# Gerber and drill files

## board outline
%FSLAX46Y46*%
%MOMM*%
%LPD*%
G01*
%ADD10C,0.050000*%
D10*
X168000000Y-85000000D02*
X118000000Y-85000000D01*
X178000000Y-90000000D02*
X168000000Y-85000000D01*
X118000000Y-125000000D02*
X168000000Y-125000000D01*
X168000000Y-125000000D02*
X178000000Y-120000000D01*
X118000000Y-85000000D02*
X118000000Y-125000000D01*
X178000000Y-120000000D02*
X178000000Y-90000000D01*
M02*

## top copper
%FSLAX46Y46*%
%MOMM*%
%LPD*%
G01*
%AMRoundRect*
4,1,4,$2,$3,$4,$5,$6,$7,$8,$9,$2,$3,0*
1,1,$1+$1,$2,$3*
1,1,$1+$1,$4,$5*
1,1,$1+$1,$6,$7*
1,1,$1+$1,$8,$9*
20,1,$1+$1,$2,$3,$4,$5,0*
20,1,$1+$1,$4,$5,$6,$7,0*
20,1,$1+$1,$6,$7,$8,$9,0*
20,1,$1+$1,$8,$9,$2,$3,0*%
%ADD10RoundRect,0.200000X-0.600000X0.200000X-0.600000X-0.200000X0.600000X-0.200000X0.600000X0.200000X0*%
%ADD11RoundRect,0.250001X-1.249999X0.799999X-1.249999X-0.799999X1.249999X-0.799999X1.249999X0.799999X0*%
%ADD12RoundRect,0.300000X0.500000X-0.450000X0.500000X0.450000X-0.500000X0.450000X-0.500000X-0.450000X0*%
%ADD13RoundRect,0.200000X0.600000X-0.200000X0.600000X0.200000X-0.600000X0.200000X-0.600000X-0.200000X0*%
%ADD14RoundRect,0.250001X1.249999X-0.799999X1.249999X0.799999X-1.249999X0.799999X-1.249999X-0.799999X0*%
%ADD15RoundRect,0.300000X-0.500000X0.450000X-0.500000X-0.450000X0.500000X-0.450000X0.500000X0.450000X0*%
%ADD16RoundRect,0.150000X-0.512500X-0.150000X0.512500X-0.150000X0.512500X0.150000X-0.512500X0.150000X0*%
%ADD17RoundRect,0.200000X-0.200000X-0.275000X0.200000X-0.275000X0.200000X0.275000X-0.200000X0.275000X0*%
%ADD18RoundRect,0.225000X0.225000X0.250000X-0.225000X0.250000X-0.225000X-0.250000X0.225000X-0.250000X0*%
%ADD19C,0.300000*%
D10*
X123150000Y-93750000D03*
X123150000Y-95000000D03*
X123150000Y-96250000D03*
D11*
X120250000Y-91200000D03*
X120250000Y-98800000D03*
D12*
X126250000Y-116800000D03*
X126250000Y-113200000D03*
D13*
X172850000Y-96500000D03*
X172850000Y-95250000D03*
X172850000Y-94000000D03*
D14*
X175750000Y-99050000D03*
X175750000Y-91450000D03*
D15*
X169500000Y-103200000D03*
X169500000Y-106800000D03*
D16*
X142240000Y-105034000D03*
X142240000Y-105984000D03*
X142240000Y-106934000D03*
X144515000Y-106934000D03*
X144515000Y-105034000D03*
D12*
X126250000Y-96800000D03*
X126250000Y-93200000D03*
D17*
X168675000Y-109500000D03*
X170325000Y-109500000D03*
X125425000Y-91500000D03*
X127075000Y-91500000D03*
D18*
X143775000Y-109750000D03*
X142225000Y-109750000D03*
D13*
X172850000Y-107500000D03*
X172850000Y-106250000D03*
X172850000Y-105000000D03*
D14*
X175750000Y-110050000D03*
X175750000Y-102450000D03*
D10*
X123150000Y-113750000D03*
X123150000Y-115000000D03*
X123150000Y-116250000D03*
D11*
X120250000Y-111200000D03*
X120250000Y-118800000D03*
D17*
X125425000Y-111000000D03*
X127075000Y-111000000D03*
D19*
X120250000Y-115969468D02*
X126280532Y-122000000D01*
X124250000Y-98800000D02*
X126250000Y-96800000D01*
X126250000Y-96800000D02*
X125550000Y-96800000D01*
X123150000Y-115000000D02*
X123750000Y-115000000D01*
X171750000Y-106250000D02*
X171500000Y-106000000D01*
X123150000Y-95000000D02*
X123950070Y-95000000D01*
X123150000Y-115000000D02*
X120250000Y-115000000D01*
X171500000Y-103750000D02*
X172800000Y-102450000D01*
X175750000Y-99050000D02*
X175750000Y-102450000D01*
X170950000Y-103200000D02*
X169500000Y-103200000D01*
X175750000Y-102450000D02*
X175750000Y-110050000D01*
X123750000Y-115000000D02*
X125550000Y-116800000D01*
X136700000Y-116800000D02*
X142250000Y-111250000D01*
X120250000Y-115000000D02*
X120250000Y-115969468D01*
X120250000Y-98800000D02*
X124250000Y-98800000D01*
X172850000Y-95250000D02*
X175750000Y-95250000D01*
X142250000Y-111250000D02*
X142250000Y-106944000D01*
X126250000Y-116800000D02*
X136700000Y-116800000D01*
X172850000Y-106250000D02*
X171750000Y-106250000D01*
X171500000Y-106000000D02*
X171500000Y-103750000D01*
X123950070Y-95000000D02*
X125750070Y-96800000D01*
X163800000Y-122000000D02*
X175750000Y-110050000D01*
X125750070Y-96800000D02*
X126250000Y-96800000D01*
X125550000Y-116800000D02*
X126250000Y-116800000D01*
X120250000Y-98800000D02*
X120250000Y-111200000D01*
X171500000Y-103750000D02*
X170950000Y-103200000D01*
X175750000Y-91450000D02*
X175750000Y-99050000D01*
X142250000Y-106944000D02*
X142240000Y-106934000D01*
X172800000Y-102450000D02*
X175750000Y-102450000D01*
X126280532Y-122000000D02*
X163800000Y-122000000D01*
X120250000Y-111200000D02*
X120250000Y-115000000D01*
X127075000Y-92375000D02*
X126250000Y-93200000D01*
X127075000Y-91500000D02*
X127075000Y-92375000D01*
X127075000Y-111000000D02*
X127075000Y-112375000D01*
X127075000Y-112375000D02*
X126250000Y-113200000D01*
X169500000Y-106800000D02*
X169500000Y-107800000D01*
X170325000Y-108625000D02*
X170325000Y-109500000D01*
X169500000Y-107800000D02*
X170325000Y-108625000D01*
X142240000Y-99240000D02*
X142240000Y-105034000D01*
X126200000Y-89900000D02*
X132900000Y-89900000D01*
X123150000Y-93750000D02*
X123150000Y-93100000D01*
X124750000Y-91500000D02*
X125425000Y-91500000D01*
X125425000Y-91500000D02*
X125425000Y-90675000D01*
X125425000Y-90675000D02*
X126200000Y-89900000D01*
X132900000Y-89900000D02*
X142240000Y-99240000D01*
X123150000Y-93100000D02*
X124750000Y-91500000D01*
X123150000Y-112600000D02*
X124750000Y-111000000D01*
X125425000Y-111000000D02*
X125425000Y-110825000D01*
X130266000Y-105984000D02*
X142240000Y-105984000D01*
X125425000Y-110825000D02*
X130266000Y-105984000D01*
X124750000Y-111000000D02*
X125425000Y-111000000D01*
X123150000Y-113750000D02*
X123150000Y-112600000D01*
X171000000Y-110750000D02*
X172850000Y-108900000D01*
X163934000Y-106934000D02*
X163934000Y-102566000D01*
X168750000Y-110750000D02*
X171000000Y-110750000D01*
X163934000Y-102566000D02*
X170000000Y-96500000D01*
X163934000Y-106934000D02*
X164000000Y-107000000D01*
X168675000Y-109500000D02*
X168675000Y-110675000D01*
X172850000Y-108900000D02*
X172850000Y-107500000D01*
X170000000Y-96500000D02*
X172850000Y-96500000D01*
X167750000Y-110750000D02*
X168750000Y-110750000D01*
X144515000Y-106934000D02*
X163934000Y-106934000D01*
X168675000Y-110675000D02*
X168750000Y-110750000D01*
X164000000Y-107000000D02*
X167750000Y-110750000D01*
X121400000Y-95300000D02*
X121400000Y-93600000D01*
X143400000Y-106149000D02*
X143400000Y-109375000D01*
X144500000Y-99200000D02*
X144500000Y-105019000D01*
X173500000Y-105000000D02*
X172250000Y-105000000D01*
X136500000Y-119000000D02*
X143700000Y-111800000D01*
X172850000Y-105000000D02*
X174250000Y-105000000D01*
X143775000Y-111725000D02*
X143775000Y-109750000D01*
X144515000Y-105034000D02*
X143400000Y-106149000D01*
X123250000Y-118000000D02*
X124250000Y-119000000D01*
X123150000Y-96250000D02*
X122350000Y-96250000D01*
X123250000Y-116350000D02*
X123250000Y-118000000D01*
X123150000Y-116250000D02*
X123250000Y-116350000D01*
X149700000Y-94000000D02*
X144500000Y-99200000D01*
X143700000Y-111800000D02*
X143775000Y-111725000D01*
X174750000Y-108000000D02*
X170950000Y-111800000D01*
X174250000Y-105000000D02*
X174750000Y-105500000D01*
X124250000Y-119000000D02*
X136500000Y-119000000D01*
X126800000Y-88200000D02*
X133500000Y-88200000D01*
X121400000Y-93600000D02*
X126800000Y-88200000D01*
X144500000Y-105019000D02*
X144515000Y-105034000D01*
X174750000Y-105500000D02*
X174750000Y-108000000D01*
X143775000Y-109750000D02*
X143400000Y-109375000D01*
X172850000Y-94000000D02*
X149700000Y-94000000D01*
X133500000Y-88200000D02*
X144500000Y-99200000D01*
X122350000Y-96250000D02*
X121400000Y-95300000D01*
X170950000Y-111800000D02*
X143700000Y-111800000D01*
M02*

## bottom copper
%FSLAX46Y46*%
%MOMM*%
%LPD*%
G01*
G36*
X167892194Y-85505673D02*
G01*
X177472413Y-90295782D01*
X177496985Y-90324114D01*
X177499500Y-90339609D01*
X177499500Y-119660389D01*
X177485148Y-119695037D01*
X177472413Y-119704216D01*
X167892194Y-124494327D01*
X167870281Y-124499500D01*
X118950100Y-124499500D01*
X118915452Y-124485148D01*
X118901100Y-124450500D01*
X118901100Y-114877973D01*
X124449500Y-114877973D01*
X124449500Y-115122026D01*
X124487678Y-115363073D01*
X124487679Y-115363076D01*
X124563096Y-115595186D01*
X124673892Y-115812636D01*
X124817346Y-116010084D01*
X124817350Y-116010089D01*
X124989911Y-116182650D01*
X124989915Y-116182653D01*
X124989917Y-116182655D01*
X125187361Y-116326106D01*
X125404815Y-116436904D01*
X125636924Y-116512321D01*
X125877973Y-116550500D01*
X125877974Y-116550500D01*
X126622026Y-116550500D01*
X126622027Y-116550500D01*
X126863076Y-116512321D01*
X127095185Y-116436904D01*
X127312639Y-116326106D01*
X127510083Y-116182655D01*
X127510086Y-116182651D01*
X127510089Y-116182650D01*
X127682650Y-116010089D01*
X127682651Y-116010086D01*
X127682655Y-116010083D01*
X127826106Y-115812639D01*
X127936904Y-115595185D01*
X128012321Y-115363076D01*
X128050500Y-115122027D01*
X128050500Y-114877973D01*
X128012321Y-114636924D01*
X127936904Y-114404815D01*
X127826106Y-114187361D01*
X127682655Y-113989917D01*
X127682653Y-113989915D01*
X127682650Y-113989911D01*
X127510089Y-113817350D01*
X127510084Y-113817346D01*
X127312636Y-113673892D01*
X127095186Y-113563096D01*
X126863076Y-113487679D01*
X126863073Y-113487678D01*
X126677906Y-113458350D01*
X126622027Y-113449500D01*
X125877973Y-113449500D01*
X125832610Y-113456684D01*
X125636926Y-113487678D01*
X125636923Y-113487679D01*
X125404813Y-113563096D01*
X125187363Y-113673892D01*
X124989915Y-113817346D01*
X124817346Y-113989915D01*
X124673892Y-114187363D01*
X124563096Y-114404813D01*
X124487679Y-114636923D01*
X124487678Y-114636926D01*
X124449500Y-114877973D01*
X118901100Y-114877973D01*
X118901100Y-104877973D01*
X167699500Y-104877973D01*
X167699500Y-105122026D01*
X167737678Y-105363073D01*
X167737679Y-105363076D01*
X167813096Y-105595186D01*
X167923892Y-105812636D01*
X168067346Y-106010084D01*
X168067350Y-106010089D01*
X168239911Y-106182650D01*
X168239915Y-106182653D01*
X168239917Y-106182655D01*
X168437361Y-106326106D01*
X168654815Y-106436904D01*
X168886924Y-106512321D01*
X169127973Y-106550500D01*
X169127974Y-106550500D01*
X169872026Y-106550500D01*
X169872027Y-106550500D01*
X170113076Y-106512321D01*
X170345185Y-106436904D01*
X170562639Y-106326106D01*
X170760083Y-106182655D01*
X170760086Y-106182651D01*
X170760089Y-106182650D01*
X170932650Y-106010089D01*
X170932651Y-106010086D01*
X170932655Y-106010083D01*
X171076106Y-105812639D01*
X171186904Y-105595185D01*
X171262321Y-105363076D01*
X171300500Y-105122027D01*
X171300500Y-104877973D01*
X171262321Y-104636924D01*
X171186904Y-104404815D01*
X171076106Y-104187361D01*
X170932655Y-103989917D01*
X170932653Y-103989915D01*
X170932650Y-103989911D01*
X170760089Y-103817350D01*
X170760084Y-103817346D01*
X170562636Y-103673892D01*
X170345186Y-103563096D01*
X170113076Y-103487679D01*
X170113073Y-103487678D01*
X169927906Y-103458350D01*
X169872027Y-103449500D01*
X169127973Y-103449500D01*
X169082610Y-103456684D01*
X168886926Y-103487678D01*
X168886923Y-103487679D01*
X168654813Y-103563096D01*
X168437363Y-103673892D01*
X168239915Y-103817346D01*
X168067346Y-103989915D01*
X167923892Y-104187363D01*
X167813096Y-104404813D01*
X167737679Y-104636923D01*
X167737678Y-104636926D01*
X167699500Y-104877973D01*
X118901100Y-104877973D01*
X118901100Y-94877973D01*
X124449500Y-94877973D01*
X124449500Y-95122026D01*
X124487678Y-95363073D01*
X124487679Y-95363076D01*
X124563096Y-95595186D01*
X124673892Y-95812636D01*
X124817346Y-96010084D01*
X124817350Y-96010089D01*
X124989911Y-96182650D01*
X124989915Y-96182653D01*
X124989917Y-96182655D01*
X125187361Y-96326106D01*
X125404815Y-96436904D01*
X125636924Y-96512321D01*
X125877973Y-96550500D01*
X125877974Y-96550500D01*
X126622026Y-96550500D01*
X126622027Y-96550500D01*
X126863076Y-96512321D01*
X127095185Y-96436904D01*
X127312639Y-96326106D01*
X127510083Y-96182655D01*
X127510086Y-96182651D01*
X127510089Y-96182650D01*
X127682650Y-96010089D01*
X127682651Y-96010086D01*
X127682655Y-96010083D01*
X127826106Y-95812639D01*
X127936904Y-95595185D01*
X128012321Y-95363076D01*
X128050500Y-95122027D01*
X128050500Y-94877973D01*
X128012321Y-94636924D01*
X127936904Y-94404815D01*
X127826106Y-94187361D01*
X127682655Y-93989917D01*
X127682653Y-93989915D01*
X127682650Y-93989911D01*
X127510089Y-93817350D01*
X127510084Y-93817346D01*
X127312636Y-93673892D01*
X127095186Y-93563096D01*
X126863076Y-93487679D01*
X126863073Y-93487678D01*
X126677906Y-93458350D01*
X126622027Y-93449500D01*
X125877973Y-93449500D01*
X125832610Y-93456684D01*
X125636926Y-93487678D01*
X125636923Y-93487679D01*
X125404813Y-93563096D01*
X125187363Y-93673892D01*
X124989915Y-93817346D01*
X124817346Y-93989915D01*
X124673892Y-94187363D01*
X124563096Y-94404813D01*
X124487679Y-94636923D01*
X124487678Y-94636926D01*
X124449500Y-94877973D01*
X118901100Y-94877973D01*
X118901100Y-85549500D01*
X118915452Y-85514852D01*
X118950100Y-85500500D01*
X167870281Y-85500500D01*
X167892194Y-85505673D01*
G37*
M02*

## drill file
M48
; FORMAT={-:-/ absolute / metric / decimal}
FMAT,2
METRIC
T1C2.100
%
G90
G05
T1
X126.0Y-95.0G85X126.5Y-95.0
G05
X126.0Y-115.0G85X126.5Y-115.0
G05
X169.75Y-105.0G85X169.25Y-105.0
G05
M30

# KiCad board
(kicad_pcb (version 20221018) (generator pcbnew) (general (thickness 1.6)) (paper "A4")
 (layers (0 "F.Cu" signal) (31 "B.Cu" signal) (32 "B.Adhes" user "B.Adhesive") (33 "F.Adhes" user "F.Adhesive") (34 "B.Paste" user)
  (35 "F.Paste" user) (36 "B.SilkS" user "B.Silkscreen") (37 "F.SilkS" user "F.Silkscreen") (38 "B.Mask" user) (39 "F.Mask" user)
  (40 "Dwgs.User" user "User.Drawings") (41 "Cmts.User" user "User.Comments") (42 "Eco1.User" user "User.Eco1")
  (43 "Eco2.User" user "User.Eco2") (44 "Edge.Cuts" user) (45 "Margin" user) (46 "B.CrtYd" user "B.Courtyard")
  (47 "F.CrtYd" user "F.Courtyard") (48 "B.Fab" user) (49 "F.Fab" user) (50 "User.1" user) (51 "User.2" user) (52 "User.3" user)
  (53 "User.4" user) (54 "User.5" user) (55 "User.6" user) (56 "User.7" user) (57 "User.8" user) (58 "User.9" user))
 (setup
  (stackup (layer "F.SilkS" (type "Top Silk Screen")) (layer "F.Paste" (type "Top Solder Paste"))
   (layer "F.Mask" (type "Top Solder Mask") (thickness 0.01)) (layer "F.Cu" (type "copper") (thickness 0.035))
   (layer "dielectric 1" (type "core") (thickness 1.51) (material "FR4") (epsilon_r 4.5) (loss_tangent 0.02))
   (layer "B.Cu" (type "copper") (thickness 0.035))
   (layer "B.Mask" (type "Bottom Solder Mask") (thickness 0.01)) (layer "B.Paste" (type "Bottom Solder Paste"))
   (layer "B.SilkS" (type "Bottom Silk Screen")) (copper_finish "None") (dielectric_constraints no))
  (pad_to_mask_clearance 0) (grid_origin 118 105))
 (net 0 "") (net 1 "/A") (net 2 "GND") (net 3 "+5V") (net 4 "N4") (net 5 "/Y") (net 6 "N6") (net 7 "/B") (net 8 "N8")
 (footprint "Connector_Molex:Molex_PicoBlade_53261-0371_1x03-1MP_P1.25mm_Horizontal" (layer "F.Cu") (at 120.75 95 -90)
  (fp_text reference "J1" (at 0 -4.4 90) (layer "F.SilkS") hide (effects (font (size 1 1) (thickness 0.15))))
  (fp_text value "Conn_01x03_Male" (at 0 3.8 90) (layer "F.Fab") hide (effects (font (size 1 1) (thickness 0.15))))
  (pad "1" smd roundrect (at -1.25 -2.4 270) (size 0.8 1.6) (layers "F.Cu" "F.Paste" "F.Mask") (roundrect_rratio 0.25) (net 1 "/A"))
  (pad "2" smd roundrect (at 0 -2.4 270) (size 0.8 1.6) (layers "F.Cu" "F.Paste" "F.Mask") (roundrect_rratio 0.25) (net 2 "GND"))
  (pad "3" smd roundrect (at 1.25 -2.4 270) (size 0.8 1.6) (layers "F.Cu" "F.Paste" "F.Mask") (roundrect_rratio 0.25) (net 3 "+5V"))
  (pad "MP" smd roundrect (at -3.8 0.5 270) (size 2.1 3) (layers "F.Cu" "F.Paste" "F.Mask") (roundrect_rratio 0.1190480952))
  (pad "MP" smd roundrect (at 3.8 0.5 270) (size 2.1 3) (layers "F.Cu" "F.Paste" "F.Mask") (roundrect_rratio 0.1190480952)))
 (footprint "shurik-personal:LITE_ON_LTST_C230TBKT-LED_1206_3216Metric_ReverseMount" (layer "F.Cu") (at 126.25 115 90)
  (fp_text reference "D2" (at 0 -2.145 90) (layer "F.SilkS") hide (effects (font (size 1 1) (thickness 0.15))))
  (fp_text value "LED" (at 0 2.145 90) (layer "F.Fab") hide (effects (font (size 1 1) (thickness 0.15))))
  (pad "" np_thru_hole oval (at 0 0 90) (size 2.1 2.6) (drill oval 2.1 2.6) (layers "F&B.Cu" "*.Mask"))
  (pad "1" smd roundrect (at -1.8 0 90) (size 1.5 1.6) (layers "F.Cu" "F.Paste" "F.Mask") (roundrect_rratio 0.2) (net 2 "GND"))
  (pad "2" smd roundrect (at 1.8 0 90) (size 1.5 1.6) (layers "F.Cu" "F.Paste" "F.Mask") (roundrect_rratio 0.2) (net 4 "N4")))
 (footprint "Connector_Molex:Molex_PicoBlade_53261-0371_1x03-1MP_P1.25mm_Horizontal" (layer "F.Cu") (at 175.25 95.25 90)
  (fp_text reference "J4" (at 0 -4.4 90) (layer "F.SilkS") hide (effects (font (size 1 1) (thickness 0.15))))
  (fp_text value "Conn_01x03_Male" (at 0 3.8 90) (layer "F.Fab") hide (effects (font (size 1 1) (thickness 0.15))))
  (pad "1" smd roundrect (at -1.25 -2.4 90) (size 0.8 1.6) (layers "F.Cu" "F.Paste" "F.Mask") (roundrect_rratio 0.25) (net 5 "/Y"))
  (pad "2" smd roundrect (at 0 -2.4 90) (size 0.8 1.6) (layers "F.Cu" "F.Paste" "F.Mask") (roundrect_rratio 0.25) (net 2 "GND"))
  (pad "3" smd roundrect (at 1.25 -2.4 90) (size 0.8 1.6) (layers "F.Cu" "F.Paste" "F.Mask") (roundrect_rratio 0.25) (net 3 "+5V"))
  (pad "MP" smd roundrect (at -3.8 0.5 90) (size 2.1 3) (layers "F.Cu" "F.Paste" "F.Mask") (roundrect_rratio 0.1190480952))
  (pad "MP" smd roundrect (at 3.8 0.5 90) (size 2.1 3) (layers "F.Cu" "F.Paste" "F.Mask") (roundrect_rratio 0.1190480952)))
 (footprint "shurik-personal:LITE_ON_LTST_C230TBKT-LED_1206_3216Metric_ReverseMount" (layer "F.Cu") (at 169.5 105 -90)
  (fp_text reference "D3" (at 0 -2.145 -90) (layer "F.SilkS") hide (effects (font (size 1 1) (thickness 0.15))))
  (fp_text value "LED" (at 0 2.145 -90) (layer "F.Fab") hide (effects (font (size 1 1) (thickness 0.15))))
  (pad "" np_thru_hole oval (at 0 0 270) (size 2.1 2.6) (drill oval 2.1 2.6) (layers "F&B.Cu" "*.Mask"))
  (pad "1" smd roundrect (at -1.8 0 270) (size 1.5 1.6) (layers "F.Cu" "F.Paste" "F.Mask") (roundrect_rratio 0.2) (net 2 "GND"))
  (pad "2" smd roundrect (at 1.8 0 270) (size 1.5 1.6) (layers "F.Cu" "F.Paste" "F.Mask") (roundrect_rratio 0.2) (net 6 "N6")))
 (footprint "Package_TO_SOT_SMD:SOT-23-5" (layer "F.Cu") (at 143.3775 105.984)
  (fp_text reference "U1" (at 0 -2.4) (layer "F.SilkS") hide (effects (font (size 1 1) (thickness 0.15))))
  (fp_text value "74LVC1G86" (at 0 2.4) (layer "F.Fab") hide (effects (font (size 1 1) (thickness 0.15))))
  (pad "1" smd roundrect (at -1.1375 -0.95) (size 1.325 0.6) (layers "F.Cu" "F.Paste" "F.Mask") (roundrect_rratio 0.25) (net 1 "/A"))
  (pad "2" smd roundrect (at -1.1375 0) (size 1.325 0.6) (layers "F.Cu" "F.Paste" "F.Mask") (roundrect_rratio 0.25) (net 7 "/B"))
  (pad "3" smd roundrect (at -1.1375 0.95) (size 1.325 0.6) (layers "F.Cu" "F.Paste" "F.Mask") (roundrect_rratio 0.25) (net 2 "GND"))
  (pad "4" smd roundrect (at 1.1375 0.95) (size 1.325 0.6) (layers "F.Cu" "F.Paste" "F.Mask") (roundrect_rratio 0.25) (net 5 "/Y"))
  (pad "5" smd roundrect (at 1.1375 -0.95) (size 1.325 0.6) (layers "F.Cu" "F.Paste" "F.Mask") (roundrect_rratio 0.25) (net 3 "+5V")))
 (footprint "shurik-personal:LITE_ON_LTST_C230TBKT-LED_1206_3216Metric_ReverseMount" (layer "F.Cu") (at 126.25 95 90)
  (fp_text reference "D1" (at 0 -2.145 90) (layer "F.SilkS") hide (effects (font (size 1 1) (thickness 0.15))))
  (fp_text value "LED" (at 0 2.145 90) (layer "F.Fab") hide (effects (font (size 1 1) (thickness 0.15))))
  (pad "" np_thru_hole oval (at 0 0 90) (size 2.1 2.6) (drill oval 2.1 2.6) (layers "F&B.Cu" "*.Mask"))
  (pad "1" smd roundrect (at -1.8 0 90) (size 1.5 1.6) (layers "F.Cu" "F.Paste" "F.Mask") (roundrect_rratio 0.2) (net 2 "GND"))
  (pad "2" smd roundrect (at 1.8 0 90) (size 1.5 1.6) (layers "F.Cu" "F.Paste" "F.Mask") (roundrect_rratio 0.2) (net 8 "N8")))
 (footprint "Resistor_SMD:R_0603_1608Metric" (layer "F.Cu") (at 169.5 109.5)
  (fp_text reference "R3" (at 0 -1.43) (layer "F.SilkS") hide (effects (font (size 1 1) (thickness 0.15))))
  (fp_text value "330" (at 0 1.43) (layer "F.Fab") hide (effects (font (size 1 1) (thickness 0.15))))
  (pad "1" smd roundrect (at -0.825 0) (size 0.8 0.95) (layers "F.Cu" "F.Paste" "F.Mask") (roundrect_rratio 0.25) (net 5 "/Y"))
  (pad "2" smd roundrect (at 0.825 0) (size 0.8 0.95) (layers "F.Cu" "F.Paste" "F.Mask") (roundrect_rratio 0.25) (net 6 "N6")))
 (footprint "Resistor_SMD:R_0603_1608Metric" (layer "F.Cu") (at 126.25 91.5)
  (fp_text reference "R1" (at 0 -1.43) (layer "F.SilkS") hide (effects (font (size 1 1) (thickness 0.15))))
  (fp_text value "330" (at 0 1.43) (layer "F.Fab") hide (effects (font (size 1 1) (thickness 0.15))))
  (pad "1" smd roundrect (at -0.825 0) (size 0.8 0.95) (layers "F.Cu" "F.Paste" "F.Mask") (roundrect_rratio 0.25) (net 1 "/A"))
  (pad "2" smd roundrect (at 0.825 0) (size 0.8 0.95) (layers "F.Cu" "F.Paste" "F.Mask") (roundrect_rratio 0.25) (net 8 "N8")))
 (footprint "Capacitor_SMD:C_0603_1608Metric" (layer "F.Cu") (at 143 109.75 180)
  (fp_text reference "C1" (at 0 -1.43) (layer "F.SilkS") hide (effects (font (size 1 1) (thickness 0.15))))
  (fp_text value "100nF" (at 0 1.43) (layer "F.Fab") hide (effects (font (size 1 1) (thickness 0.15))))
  (pad "1" smd roundrect (at -0.775 0 180) (size 0.9 0.95) (layers "F.Cu" "F.Paste" "F.Mask") (roundrect_rratio 0.25) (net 3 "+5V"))
  (pad "2" smd roundrect (at 0.775 0 180) (size 0.9 0.95) (layers "F.Cu" "F.Paste" "F.Mask") (roundrect_rratio 0.25) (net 2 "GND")))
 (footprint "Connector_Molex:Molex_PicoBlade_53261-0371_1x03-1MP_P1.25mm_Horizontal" (layer "F.Cu") (at 175.25 106.25 90)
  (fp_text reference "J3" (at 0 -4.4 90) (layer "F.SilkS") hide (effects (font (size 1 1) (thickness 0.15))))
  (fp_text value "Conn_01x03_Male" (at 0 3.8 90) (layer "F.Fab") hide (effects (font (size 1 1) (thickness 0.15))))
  (pad "1" smd roundrect (at -1.25 -2.4 90) (size 0.8 1.6) (layers "F.Cu" "F.Paste" "F.Mask") (roundrect_rratio 0.25) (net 5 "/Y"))
  (pad "2" smd roundrect (at 0 -2.4 90) (size 0.8 1.6) (layers "F.Cu" "F.Paste" "F.Mask") (roundrect_rratio 0.25) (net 2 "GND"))
  (pad "3" smd roundrect (at 1.25 -2.4 90) (size 0.8 1.6) (layers "F.Cu" "F.Paste" "F.Mask") (roundrect_rratio 0.25) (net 3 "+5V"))
  (pad "MP" smd roundrect (at -3.8 0.5 90) (size 2.1 3) (layers "F.Cu" "F.Paste" "F.Mask") (roundrect_rratio 0.1190480952))
  (pad "MP" smd roundrect (at 3.8 0.5 90) (size 2.1 3) (layers "F.Cu" "F.Paste" "F.Mask") (roundrect_rratio 0.1190480952)))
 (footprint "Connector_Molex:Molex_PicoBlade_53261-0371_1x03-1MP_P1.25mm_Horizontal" (layer "F.Cu") (at 120.75 115 -90)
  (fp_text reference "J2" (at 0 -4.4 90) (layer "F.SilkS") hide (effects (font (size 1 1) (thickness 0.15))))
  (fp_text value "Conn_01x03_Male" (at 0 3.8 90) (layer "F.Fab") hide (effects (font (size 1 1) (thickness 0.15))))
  (pad "1" smd roundrect (at -1.25 -2.4 270) (size 0.8 1.6) (layers "F.Cu" "F.Paste" "F.Mask") (roundrect_rratio 0.25) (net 7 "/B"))
  (pad "2" smd roundrect (at 0 -2.4 270) (size 0.8 1.6) (layers "F.Cu" "F.Paste" "F.Mask") (roundrect_rratio 0.25) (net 2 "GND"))
  (pad "3" smd roundrect (at 1.25 -2.4 270) (size 0.8 1.6) (layers "F.Cu" "F.Paste" "F.Mask") (roundrect_rratio 0.25) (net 3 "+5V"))
  (pad "MP" smd roundrect (at -3.8 0.5 270) (size 2.1 3) (layers "F.Cu" "F.Paste" "F.Mask") (roundrect_rratio 0.1190480952))
  (pad "MP" smd roundrect (at 3.8 0.5 270) (size 2.1 3) (layers "F.Cu" "F.Paste" "F.Mask") (roundrect_rratio 0.1190480952)))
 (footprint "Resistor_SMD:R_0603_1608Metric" (layer "F.Cu") (at 126.25 111)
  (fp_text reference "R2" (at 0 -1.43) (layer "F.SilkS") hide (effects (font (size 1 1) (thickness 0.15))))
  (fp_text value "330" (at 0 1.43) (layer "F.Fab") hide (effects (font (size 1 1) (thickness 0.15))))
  (pad "1" smd roundrect (at -0.825 0) (size 0.8 0.95) (layers "F.Cu" "F.Paste" "F.Mask") (roundrect_rratio 0.25) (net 7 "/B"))
  (pad "2" smd roundrect (at 0.825 0) (size 0.8 0.95) (layers "F.Cu" "F.Paste" "F.Mask") (roundrect_rratio 0.25) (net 4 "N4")))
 (gr_line (start 168 85) (end 118 85) (stroke (width 0.05) (type solid)) (layer "Edge.Cuts"))
 (gr_line (start 178 90) (end 168 85) (stroke (width 0.05) (type solid)) (layer "Edge.Cuts"))
 (gr_line (start 118 125) (end 168 125) (stroke (width 0.05) (type solid)) (layer "Edge.Cuts"))
 (gr_line (start 168 125) (end 178 120) (stroke (width 0.05) (type solid)) (layer "Edge.Cuts"))
 (gr_line (start 118 85) (end 118 125) (stroke (width 0.05) (type solid)) (layer "Edge.Cuts"))
 (gr_line (start 178 120) (end 178 90) (stroke (width 0.05) (type solid)) (layer "Edge.Cuts"))
 (segment (start 120.25 115.969468) (end 126.280532 122) (width 0.3) (layer "F.Cu") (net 2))
 (segment (start 124.25 98.8) (end 126.25 96.8) (width 0.3) (layer "F.Cu") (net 2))
 (segment (start 126.25 96.8) (end 125.55 96.8) (width 0.3) (layer "F.Cu") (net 2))
 (segment (start 123.15 115) (end 123.75 115) (width 0.3) (layer "F.Cu") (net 2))
 (segment (start 171.75 106.25) (end 171.5 106) (width 0.3) (layer "F.Cu") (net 2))
 (segment (start 123.15 95) (end 123.95007 95) (width 0.3) (layer "F.Cu") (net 2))
 (segment (start 123.15 115) (end 120.25 115) (width 0.3) (layer "F.Cu") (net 2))
 (segment (start 171.5 103.75) (end 172.8 102.45) (width 0.3) (layer "F.Cu") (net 2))
 (segment (start 175.75 99.05) (end 175.75 102.45) (width 0.3) (layer "F.Cu") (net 2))
 (segment (start 170.95 103.2) (end 169.5 103.2) (width 0.3) (layer "F.Cu") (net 2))
 (segment (start 175.75 102.45) (end 175.75 110.05) (width 0.3) (layer "F.Cu") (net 2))
 (segment (start 123.75 115) (end 125.55 116.8) (width 0.3) (layer "F.Cu") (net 2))
 (segment (start 136.7 116.8) (end 142.25 111.25) (width 0.3) (layer "F.Cu") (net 2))
 (segment (start 120.25 115) (end 120.25 115.969468) (width 0.3) (layer "F.Cu") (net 2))
 (segment (start 120.25 98.8) (end 124.25 98.8) (width 0.3) (layer "F.Cu") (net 2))
 (segment (start 172.85 95.25) (end 175.75 95.25) (width 0.3) (layer "F.Cu") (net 2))
 (segment (start 142.25 111.25) (end 142.25 106.944) (width 0.3) (layer "F.Cu") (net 2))
 (segment (start 126.25 116.8) (end 136.7 116.8) (width 0.3) (layer "F.Cu") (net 2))
 (segment (start 172.85 106.25) (end 171.75 106.25) (width 0.3) (layer "F.Cu") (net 2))
 (segment (start 171.5 106) (end 171.5 103.75) (width 0.3) (layer "F.Cu") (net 2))
 (segment (start 123.95007 95) (end 125.75007 96.8) (width 0.3) (layer "F.Cu") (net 2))
 (segment (start 163.8 122) (end 175.75 110.05) (width 0.3) (layer "F.Cu") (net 2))
 (segment (start 125.75007 96.8) (end 126.25 96.8) (width 0.3) (layer "F.Cu") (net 2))
 (segment (start 125.55 116.8) (end 126.25 116.8) (width 0.3) (layer "F.Cu") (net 2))
 (segment (start 120.25 98.8) (end 120.25 111.2) (width 0.3) (layer "F.Cu") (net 2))
 (segment (start 171.5 103.75) (end 170.95 103.2) (width 0.3) (layer "F.Cu") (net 2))
 (segment (start 175.75 91.45) (end 175.75 99.05) (width 0.3) (layer "F.Cu") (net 2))
 (segment (start 142.25 106.944) (end 142.24 106.934) (width 0.3) (layer "F.Cu") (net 2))
 (segment (start 172.8 102.45) (end 175.75 102.45) (width 0.3) (layer "F.Cu") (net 2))
 (segment (start 126.280532 122) (end 163.8 122) (width 0.3) (layer "F.Cu") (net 2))
 (segment (start 120.25 111.2) (end 120.25 115) (width 0.3) (layer "F.Cu") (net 2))
 (segment (start 127.075 92.375) (end 126.25 93.2) (width 0.3) (layer "F.Cu") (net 8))
 (segment (start 127.075 91.5) (end 127.075 92.375) (width 0.3) (layer "F.Cu") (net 8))
 (segment (start 127.075 111) (end 127.075 112.375) (width 0.3) (layer "F.Cu") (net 4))
 (segment (start 127.075 112.375) (end 126.25 113.2) (width 0.3) (layer "F.Cu") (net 4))
 (segment (start 169.5 106.8) (end 169.5 107.8) (width 0.3) (layer "F.Cu") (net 6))
 (segment (start 170.325 108.625) (end 170.325 109.5) (width 0.3) (layer "F.Cu") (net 6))
 (segment (start 169.5 107.8) (end 170.325 108.625) (width 0.3) (layer "F.Cu") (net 6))
 (segment (start 142.24 99.24) (end 142.24 105.034) (width 0.3) (layer "F.Cu") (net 1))
 (segment (start 126.2 89.9) (end 132.9 89.9) (width 0.3) (layer "F.Cu") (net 1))
 (segment (start 123.15 93.75) (end 123.15 93.1) (width 0.3) (layer "F.Cu") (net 1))
 (segment (start 124.75 91.5) (end 125.425 91.5) (width 0.3) (layer "F.Cu") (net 1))
 (segment (start 125.425 91.5) (end 125.425 90.675) (width 0.3) (layer "F.Cu") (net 1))
 (segment (start 125.425 90.675) (end 126.2 89.9) (width 0.3) (layer "F.Cu") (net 1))
 (segment (start 132.9 89.9) (end 142.24 99.24) (width 0.3) (layer "F.Cu") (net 1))
 (segment (start 123.15 93.1) (end 124.75 91.5) (width 0.3) (layer "F.Cu") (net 1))
 (segment (start 123.15 112.6) (end 124.75 111) (width 0.3) (layer "F.Cu") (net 7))
 (segment (start 125.425 111) (end 125.425 110.825) (width 0.3) (layer "F.Cu") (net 7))
 (segment (start 130.266 105.984) (end 142.24 105.984) (width 0.3) (layer "F.Cu") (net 7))
 (segment (start 125.425 110.825) (end 130.266 105.984) (width 0.3) (layer "F.Cu") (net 7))
 (segment (start 124.75 111) (end 125.425 111) (width 0.3) (layer "F.Cu") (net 7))
 (segment (start 123.15 113.75) (end 123.15 112.6) (width 0.3) (layer "F.Cu") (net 7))
 (segment (start 171 110.75) (end 172.85 108.9) (width 0.3) (layer "F.Cu") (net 5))
 (segment (start 163.934 106.934) (end 163.934 102.566) (width 0.3) (layer "F.Cu") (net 5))
 (segment (start 168.75 110.75) (end 171 110.75) (width 0.3) (layer "F.Cu") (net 5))
 (segment (start 163.934 102.566) (end 170 96.5) (width 0.3) (layer "F.Cu") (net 5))
 (segment (start 163.934 106.934) (end 164 107) (width 0.3) (layer "F.Cu") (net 5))
 (segment (start 168.675 109.5) (end 168.675 110.675) (width 0.3) (layer "F.Cu") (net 5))
 (segment (start 172.85 108.9) (end 172.85 107.5) (width 0.3) (layer "F.Cu") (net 5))
 (segment (start 170 96.5) (end 172.85 96.5) (width 0.3) (layer "F.Cu") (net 5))
 (segment (start 167.75 110.75) (end 168.75 110.75) (width 0.3) (layer "F.Cu") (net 5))
 (segment (start 144.515 106.934) (end 163.934 106.934) (width 0.3) (layer "F.Cu") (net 5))
 (segment (start 168.675 110.675) (end 168.75 110.75) (width 0.3) (layer "F.Cu") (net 5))
 (segment (start 164 107) (end 167.75 110.75) (width 0.3) (layer "F.Cu") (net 5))
 (segment (start 121.4 95.3) (end 121.4 93.6) (width 0.3) (layer "F.Cu") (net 3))
 (segment (start 143.4 106.149) (end 143.4 109.375) (width 0.3) (layer "F.Cu") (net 3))
 (segment (start 144.5 99.2) (end 144.5 105.019) (width 0.3) (layer "F.Cu") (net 3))
 (segment (start 173.5 105) (end 172.25 105) (width 0.3) (layer "F.Cu") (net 3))
 (segment (start 136.5 119) (end 143.7 111.8) (width 0.3) (layer "F.Cu") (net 3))
 (segment (start 172.85 105) (end 174.25 105) (width 0.3) (layer "F.Cu") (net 3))
 (segment (start 143.775 111.725) (end 143.775 109.75) (width 0.3) (layer "F.Cu") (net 3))
 (segment (start 144.515 105.034) (end 143.4 106.149) (width 0.3) (layer "F.Cu") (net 3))
 (segment (start 123.25 118) (end 124.25 119) (width 0.3) (layer "F.Cu") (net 3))
 (segment (start 123.15 96.25) (end 122.35 96.25) (width 0.3) (layer "F.Cu") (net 3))
 (segment (start 123.25 116.35) (end 123.25 118) (width 0.3) (layer "F.Cu") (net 3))
 (segment (start 123.15 116.25) (end 123.25 116.35) (width 0.3) (layer "F.Cu") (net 3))
 (segment (start 149.7 94) (end 144.5 99.2) (width 0.3) (layer "F.Cu") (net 3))
 (segment (start 143.7 111.8) (end 143.775 111.725) (width 0.3) (layer "F.Cu") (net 3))
 (segment (start 174.75 108) (end 170.95 111.8) (width 0.3) (layer "F.Cu") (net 3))
 (segment (start 174.25 105) (end 174.75 105.5) (width 0.3) (layer "F.Cu") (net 3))
 (segment (start 124.25 119) (end 136.5 119) (width 0.3) (layer "F.Cu") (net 3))
 (segment (start 126.8 88.2) (end 133.5 88.2) (width 0.3) (layer "F.Cu") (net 3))
 (segment (start 121.4 93.6) (end 126.8 88.2) (width 0.3) (layer "F.Cu") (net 3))
 (segment (start 144.5 105.019) (end 144.515 105.034) (width 0.3) (layer "F.Cu") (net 3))
 (segment (start 174.75 105.5) (end 174.75 108) (width 0.3) (layer "F.Cu") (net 3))
 (segment (start 143.775 109.75) (end 143.4 109.375) (width 0.3) (layer "F.Cu") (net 3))
 (segment (start 172.85 94) (end 149.7 94) (width 0.3) (layer "F.Cu") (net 3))
 (segment (start 133.5 88.2) (end 144.5 99.2) (width 0.3) (layer "F.Cu") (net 3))
 (segment (start 122.35 96.25) (end 121.4 95.3) (width 0.3) (layer "F.Cu") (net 3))
 (segment (start 170.95 111.8) (end 143.7 111.8) (width 0.3) (layer "F.Cu") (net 3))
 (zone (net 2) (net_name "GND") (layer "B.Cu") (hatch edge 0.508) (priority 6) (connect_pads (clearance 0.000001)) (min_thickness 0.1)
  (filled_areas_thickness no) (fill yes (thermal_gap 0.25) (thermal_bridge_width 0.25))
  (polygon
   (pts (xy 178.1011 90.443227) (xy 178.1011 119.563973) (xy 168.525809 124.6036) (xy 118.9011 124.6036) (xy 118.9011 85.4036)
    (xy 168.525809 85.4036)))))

